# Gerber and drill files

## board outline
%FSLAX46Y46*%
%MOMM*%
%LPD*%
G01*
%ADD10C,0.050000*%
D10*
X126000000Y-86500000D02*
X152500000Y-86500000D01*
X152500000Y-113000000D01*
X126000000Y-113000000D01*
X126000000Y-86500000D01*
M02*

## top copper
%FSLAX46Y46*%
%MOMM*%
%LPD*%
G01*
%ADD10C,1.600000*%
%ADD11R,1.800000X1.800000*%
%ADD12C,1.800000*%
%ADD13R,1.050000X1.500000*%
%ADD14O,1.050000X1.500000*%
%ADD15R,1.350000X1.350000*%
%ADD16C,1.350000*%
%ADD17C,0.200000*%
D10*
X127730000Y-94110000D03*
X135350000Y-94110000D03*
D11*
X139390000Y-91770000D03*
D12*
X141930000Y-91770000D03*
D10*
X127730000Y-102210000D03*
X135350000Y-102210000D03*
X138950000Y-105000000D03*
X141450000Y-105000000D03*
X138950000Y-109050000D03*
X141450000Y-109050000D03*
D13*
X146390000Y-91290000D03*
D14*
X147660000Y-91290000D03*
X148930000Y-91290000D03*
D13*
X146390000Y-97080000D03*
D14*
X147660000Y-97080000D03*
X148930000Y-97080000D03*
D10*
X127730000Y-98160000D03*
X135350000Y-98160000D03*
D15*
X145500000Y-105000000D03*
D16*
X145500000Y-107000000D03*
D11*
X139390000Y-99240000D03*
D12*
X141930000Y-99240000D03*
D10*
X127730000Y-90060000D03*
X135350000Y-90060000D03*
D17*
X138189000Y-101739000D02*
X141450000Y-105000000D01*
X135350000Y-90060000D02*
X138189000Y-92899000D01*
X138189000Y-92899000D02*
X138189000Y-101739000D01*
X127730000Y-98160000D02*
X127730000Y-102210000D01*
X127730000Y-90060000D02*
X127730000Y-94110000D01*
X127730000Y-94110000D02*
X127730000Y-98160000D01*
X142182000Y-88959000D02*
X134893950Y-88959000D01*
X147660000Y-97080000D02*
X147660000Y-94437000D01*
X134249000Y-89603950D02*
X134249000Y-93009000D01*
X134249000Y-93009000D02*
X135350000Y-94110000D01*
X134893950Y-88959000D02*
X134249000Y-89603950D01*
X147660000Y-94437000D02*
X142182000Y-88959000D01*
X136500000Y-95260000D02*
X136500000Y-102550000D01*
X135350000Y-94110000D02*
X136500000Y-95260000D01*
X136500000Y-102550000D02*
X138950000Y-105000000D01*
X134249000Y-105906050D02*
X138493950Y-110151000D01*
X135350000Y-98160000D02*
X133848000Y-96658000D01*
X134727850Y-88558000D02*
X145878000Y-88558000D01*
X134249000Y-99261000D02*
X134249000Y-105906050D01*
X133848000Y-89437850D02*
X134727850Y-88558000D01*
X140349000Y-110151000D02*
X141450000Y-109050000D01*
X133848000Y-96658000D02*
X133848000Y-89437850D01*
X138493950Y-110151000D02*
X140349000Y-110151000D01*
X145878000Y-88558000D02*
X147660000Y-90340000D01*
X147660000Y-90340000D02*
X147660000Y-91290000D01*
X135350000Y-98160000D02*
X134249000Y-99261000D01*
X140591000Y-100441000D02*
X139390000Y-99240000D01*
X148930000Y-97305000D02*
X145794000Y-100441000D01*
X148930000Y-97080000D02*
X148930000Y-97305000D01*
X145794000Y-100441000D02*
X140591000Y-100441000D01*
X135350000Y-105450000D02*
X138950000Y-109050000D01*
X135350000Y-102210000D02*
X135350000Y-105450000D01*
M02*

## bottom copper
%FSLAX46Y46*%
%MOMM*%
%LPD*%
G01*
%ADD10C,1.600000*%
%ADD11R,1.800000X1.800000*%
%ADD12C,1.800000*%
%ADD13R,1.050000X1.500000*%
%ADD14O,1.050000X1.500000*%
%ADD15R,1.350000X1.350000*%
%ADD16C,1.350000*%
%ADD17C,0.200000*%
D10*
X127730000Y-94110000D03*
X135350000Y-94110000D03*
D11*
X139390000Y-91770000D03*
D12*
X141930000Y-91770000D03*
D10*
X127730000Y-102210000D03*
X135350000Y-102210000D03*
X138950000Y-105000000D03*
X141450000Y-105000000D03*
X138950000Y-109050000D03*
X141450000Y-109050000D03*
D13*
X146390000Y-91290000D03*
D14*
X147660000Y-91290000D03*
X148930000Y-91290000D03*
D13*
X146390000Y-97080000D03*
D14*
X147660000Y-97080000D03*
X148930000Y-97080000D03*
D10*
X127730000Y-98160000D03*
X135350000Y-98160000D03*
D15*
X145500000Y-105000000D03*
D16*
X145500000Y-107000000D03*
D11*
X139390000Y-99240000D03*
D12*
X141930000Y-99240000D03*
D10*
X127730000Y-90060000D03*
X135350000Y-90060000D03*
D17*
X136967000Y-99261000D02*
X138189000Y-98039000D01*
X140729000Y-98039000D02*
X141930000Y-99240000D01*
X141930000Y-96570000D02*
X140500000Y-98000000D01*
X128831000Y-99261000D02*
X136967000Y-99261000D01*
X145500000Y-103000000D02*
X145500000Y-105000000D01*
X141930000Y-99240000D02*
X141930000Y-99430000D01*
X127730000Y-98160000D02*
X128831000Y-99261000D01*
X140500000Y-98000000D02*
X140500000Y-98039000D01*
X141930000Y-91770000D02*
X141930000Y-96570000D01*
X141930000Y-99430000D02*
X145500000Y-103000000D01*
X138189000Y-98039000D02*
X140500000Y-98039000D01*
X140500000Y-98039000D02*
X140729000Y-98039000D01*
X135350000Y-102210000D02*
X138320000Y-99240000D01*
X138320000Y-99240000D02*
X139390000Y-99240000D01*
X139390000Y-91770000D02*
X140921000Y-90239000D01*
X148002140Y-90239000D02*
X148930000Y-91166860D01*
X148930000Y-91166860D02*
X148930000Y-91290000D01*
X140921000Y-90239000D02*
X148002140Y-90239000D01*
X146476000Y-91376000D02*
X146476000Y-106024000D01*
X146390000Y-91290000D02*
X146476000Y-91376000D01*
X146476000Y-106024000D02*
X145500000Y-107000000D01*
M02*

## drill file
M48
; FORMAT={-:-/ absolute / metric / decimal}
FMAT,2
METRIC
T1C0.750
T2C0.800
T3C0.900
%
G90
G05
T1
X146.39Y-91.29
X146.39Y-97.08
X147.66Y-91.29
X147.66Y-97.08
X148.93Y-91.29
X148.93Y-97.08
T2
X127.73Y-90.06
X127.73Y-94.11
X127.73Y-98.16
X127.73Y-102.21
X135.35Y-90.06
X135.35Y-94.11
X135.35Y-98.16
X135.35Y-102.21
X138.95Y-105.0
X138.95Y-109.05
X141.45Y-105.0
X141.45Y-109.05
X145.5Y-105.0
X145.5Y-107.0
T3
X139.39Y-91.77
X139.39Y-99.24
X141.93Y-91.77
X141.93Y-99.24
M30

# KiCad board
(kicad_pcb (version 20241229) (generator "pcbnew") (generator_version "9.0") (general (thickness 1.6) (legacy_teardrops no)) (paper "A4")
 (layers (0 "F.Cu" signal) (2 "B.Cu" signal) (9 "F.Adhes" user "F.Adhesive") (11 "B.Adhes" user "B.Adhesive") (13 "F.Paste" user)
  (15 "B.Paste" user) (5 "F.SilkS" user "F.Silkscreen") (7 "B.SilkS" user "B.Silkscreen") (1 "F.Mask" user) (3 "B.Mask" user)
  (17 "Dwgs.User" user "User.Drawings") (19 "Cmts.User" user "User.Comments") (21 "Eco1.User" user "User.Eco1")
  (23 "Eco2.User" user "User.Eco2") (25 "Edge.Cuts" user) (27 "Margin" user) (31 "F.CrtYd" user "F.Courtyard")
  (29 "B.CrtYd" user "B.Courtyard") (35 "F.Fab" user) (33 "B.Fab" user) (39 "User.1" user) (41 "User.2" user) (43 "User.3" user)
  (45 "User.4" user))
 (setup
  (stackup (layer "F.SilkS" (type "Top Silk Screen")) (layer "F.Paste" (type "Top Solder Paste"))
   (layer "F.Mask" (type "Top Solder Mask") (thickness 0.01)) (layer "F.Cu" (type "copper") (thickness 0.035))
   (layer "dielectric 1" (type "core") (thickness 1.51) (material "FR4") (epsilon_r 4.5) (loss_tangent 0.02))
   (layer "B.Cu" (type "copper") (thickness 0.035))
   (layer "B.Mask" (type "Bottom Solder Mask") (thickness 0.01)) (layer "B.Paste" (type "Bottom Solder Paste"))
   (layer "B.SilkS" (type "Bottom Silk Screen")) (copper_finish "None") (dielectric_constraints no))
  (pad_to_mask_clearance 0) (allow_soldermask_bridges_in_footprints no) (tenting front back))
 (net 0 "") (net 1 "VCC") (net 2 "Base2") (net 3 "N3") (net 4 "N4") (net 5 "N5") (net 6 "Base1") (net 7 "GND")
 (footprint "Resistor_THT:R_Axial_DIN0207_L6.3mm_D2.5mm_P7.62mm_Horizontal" (layer "F.Cu") (at 127.73 94.11)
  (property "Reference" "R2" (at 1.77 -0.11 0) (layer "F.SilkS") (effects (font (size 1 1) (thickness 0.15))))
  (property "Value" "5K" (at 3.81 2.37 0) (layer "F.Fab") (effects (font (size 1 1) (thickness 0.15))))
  (pad "1" thru_hole circle (at 0 0) (size 1.6 1.6) (drill 0.8) (layers "*.Cu" "*.Mask") (remove_unused_layers no) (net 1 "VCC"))
  (pad "2" thru_hole circle (at 7.62 0) (size 1.6 1.6) (drill 0.8) (layers "*.Cu" "*.Mask") (remove_unused_layers no) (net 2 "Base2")))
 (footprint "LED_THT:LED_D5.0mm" (layer "F.Cu") (at 139.39 91.77)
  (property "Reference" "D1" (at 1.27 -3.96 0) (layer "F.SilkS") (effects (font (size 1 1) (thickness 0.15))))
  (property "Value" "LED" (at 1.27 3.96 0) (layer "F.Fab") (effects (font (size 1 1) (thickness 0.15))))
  (pad "1" thru_hole rect (at 0 0) (size 1.8 1.8) (drill 0.9) (layers "*.Cu" "*.Mask") (remove_unused_layers no) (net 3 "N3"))
  (pad "2" thru_hole circle (at 2.54 0) (size 1.8 1.8) (drill 0.9) (layers "*.Cu" "*.Mask") (remove_unused_layers no) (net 1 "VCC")))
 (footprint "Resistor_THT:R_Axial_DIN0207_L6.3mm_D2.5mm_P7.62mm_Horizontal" (layer "F.Cu") (at 127.73 102.21)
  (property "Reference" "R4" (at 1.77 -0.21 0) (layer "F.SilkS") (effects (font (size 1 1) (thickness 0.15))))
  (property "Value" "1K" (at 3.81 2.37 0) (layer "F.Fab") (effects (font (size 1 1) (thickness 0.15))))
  (pad "1" thru_hole circle (at 0 0) (size 1.6 1.6) (drill 0.8) (layers "*.Cu" "*.Mask") (remove_unused_layers no) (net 1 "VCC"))
  (pad "2" thru_hole circle (at 7.62 0) (size 1.6 1.6) (drill 0.8) (layers "*.Cu" "*.Mask") (remove_unused_layers no) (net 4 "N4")))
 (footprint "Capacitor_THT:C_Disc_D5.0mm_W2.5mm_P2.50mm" (layer "F.Cu") (at 138.95 105)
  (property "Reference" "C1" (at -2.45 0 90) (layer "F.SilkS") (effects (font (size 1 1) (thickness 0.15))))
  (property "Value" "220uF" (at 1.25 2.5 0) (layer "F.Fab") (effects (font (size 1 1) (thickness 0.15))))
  (pad "1" thru_hole circle (at 0 0) (size 1.6 1.6) (drill 0.8) (layers "*.Cu" "*.Mask") (remove_unused_layers no) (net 2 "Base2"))
  (pad "2" thru_hole circle (at 2.5 0) (size 1.6 1.6) (drill 0.8) (layers "*.Cu" "*.Mask") (remove_unused_layers no) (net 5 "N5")))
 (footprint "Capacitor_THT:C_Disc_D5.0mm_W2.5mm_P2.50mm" (layer "F.Cu") (at 138.95 109.05)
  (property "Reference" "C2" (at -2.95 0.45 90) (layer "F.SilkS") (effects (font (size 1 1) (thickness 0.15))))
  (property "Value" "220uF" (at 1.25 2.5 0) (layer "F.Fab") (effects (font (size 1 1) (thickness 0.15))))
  (pad "1" thru_hole circle (at 0 0) (size 1.6 1.6) (drill 0.8) (layers "*.Cu" "*.Mask") (remove_unused_layers no) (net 4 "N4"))
  (pad "2" thru_hole circle (at 2.5 0) (size 1.6 1.6) (drill 0.8) (layers "*.Cu" "*.Mask") (remove_unused_layers no) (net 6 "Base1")))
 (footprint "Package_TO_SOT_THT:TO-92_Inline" (layer "F.Cu") (at 146.39 91.29)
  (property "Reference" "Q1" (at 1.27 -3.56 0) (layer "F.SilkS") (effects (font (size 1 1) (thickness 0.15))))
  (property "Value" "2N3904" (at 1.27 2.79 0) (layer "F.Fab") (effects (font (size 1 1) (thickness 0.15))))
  (pad "1" thru_hole rect (at 0 0) (size 1.05 1.5) (drill 0.75) (layers "*.Cu" "*.Mask") (remove_unused_layers no) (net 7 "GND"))
  (pad "2" thru_hole oval (at 1.27 0) (size 1.05 1.5) (drill 0.75) (layers "*.Cu" "*.Mask") (remove_unused_layers no) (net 6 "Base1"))
  (pad "3" thru_hole oval (at 2.54 0) (size 1.05 1.5) (drill 0.75) (layers "*.Cu" "*.Mask") (remove_unused_layers no) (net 3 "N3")))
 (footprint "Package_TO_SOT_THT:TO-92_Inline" (layer "F.Cu") (at 146.39 97.08)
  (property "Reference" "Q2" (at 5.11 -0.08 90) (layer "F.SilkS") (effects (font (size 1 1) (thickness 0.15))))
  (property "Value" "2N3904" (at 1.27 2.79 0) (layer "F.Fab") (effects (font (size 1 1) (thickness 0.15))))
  (pad "1" thru_hole rect (at 0 0) (size 1.05 1.5) (drill 0.75) (layers "*.Cu" "*.Mask") (remove_unused_layers no) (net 7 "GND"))
  (pad "2" thru_hole oval (at 1.27 0) (size 1.05 1.5) (drill 0.75) (layers "*.Cu" "*.Mask") (remove_unused_layers no) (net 2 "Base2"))
  (pad "3" thru_hole oval (at 2.54 0) (size 1.05 1.5) (drill 0.75) (layers "*.Cu" "*.Mask") (remove_unused_layers no) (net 4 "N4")))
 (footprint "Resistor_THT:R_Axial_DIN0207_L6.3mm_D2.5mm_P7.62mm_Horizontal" (layer "F.Cu") (at 127.73 98.16)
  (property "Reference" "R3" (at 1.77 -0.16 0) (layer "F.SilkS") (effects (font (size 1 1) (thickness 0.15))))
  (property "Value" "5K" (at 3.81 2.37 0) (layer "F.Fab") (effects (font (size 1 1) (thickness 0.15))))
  (pad "1" thru_hole circle (at 0 0) (size 1.6 1.6) (drill 0.8) (layers "*.Cu" "*.Mask") (remove_unused_layers no) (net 1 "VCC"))
  (pad "2" thru_hole circle (at 7.62 0) (size 1.6 1.6) (drill 0.8) (layers "*.Cu" "*.Mask") (remove_unused_layers no) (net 6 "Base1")))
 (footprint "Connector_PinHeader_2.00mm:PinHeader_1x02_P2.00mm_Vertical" (layer "F.Cu") (at 145.5 105)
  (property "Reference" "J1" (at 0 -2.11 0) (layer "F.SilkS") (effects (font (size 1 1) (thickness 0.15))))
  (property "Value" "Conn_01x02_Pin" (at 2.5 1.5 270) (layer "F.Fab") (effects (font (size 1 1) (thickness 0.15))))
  (pad "1" thru_hole rect (at 0 0) (size 1.35 1.35) (drill 0.8) (layers "*.Cu" "*.Mask") (remove_unused_layers no) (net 1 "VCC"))
  (pad "2" thru_hole circle (at 0 2) (size 1.35 1.35) (drill 0.8) (layers "*.Cu" "*.Mask") (remove_unused_layers no) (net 7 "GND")))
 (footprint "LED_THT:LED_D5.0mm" (layer "F.Cu") (at 139.39 99.24)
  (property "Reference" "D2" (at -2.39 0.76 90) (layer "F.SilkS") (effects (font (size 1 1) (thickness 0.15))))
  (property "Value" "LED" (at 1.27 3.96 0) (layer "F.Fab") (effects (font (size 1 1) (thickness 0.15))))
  (pad "1" thru_hole rect (at 0 0) (size 1.8 1.8) (drill 0.9) (layers "*.Cu" "*.Mask") (remove_unused_layers no) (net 4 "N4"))
  (pad "2" thru_hole circle (at 2.54 0) (size 1.8 1.8) (drill 0.9) (layers "*.Cu" "*.Mask") (remove_unused_layers no) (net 1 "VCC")))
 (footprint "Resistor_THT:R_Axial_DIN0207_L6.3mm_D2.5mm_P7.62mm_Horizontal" (layer "F.Cu") (at 127.73 90.06)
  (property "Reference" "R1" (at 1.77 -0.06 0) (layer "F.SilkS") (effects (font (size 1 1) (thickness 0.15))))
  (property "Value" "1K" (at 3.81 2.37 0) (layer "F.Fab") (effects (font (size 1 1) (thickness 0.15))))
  (pad "1" thru_hole circle (at 0 0) (size 1.6 1.6) (drill 0.8) (layers "*.Cu" "*.Mask") (remove_unused_layers no) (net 1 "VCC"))
  (pad "2" thru_hole circle (at 7.62 0) (size 1.6 1.6) (drill 0.8) (layers "*.Cu" "*.Mask") (remove_unused_layers no) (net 5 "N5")))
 (gr_rect (start 126 86.5) (end 152.5 113) (stroke (width 0.05) (type default)) (fill no) (layer "Edge.Cuts"))
 (segment (start 138.189 101.739) (end 141.45 105) (width 0.2) (layer "F.Cu") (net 5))
 (segment (start 135.35 90.06) (end 138.189 92.899) (width 0.2) (layer "F.Cu") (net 5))
 (segment (start 138.189 92.899) (end 138.189 101.739) (width 0.2) (layer "F.Cu") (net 5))
 (segment (start 127.73 98.16) (end 127.73 102.21) (width 0.2) (layer "F.Cu") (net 1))
 (segment (start 127.73 90.06) (end 127.73 94.11) (width 0.2) (layer "F.Cu") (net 1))
 (segment (start 127.73 94.11) (end 127.73 98.16) (width 0.2) (layer "F.Cu") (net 1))
 (segment (start 136.967 99.261) (end 138.189 98.039) (width 0.2) (layer "B.Cu") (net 1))
 (segment (start 140.729 98.039) (end 141.93 99.24) (width 0.2) (layer "B.Cu") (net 1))
 (segment (start 141.93 96.57) (end 140.5 98) (width 0.2) (layer "B.Cu") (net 1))
 (segment (start 128.831 99.261) (end 136.967 99.261) (width 0.2) (layer "B.Cu") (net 1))
 (segment (start 145.5 103) (end 145.5 105) (width 0.2) (layer "B.Cu") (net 1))
 (segment (start 141.93 99.24) (end 141.93 99.43) (width 0.2) (layer "B.Cu") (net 1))
 (segment (start 127.73 98.16) (end 128.831 99.261) (width 0.2) (layer "B.Cu") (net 1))
 (segment (start 140.5 98) (end 140.5 98.039) (width 0.2) (layer "B.Cu") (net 1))
 (segment (start 141.93 91.77) (end 141.93 96.57) (width 0.2) (layer "B.Cu") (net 1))
 (segment (start 141.93 99.43) (end 145.5 103) (width 0.2) (layer "B.Cu") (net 1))
 (segment (start 138.189 98.039) (end 140.5 98.039) (width 0.2) (layer "B.Cu") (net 1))
 (segment (start 140.5 98.039) (end 140.729 98.039) (width 0.2) (layer "B.Cu") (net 1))
 (segment (start 142.182 88.959) (end 134.89395 88.959) (width 0.2) (layer "F.Cu") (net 2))
 (segment (start 147.66 97.08) (end 147.66 94.437) (width 0.2) (layer "F.Cu") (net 2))
 (segment (start 134.249 89.60395) (end 134.249 93.009) (width 0.2) (layer "F.Cu") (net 2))
 (segment (start 134.249 93.009) (end 135.35 94.11) (width 0.2) (layer "F.Cu") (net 2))
 (segment (start 134.89395 88.959) (end 134.249 89.60395) (width 0.2) (layer "F.Cu") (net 2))
 (segment (start 147.66 94.437) (end 142.182 88.959) (width 0.2) (layer "F.Cu") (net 2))
 (segment (start 136.5 95.26) (end 136.5 102.55) (width 0.2) (layer "F.Cu") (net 2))
 (segment (start 135.35 94.11) (end 136.5 95.26) (width 0.2) (layer "F.Cu") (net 2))
 (segment (start 136.5 102.55) (end 138.95 105) (width 0.2) (layer "F.Cu") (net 2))
 (segment (start 134.249 105.90605) (end 138.49395 110.151) (width 0.2) (layer "F.Cu") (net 6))
 (segment (start 135.35 98.16) (end 133.848 96.658) (width 0.2) (layer "F.Cu") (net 6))
 (segment (start 134.72785 88.558) (end 145.878 88.558) (width 0.2) (layer "F.Cu") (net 6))
 (segment (start 134.249 99.261) (end 134.249 105.90605) (width 0.2) (layer "F.Cu") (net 6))
 (segment (start 133.848 89.43785) (end 134.72785 88.558) (width 0.2) (layer "F.Cu") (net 6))
 (segment (start 140.349 110.151) (end 141.45 109.05) (width 0.2) (layer "F.Cu") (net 6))
 (segment (start 133.848 96.658) (end 133.848 89.43785) (width 0.2) (layer "F.Cu") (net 6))
 (segment (start 138.49395 110.151) (end 140.349 110.151) (width 0.2) (layer "F.Cu") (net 6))
 (segment (start 145.878 88.558) (end 147.66 90.34) (width 0.2) (layer "F.Cu") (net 6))
 (segment (start 147.66 90.34) (end 147.66 91.29) (width 0.2) (layer "F.Cu") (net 6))
 (segment (start 135.35 98.16) (end 134.249 99.261) (width 0.2) (layer "F.Cu") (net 6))
 (segment (start 140.591 100.441) (end 139.39 99.24) (width 0.2) (layer "F.Cu") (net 4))
 (segment (start 148.93 97.305) (end 145.794 100.441) (width 0.2) (layer "F.Cu") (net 4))
 (segment (start 148.93 97.08) (end 148.93 97.305) (width 0.2) (layer "F.Cu") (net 4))
 (segment (start 145.794 100.441) (end 140.591 100.441) (width 0.2) (layer "F.Cu") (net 4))
 (segment (start 135.35 105.45) (end 138.95 109.05) (width 0.2) (layer "F.Cu") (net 4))
 (segment (start 135.35 102.21) (end 135.35 105.45) (width 0.2) (layer "F.Cu") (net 4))
 (segment (start 135.35 102.21) (end 138.32 99.24) (width 0.2) (layer "B.Cu") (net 4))
 (segment (start 138.32 99.24) (end 139.39 99.24) (width 0.2) (layer "B.Cu") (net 4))
 (segment (start 139.39 91.77) (end 140.921 90.239) (width 0.2) (layer "B.Cu") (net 3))
 (segment (start 148.00214 90.239) (end 148.93 91.16686) (width 0.2) (layer "B.Cu") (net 3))
 (segment (start 148.93 91.16686) (end 148.93 91.29) (width 0.2) (layer "B.Cu") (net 3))
 (segment (start 140.921 90.239) (end 148.00214 90.239) (width 0.2) (layer "B.Cu") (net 3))
 (segment (start 146.476 91.376) (end 146.476 106.024) (width 0.2) (layer "B.Cu") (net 7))
 (segment (start 146.39 91.29) (end 146.476 91.376) (width 0.2) (layer "B.Cu") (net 7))
 (segment (start 146.476 106.024) (end 145.5 107) (width 0.2) (layer "B.Cu") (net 7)))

